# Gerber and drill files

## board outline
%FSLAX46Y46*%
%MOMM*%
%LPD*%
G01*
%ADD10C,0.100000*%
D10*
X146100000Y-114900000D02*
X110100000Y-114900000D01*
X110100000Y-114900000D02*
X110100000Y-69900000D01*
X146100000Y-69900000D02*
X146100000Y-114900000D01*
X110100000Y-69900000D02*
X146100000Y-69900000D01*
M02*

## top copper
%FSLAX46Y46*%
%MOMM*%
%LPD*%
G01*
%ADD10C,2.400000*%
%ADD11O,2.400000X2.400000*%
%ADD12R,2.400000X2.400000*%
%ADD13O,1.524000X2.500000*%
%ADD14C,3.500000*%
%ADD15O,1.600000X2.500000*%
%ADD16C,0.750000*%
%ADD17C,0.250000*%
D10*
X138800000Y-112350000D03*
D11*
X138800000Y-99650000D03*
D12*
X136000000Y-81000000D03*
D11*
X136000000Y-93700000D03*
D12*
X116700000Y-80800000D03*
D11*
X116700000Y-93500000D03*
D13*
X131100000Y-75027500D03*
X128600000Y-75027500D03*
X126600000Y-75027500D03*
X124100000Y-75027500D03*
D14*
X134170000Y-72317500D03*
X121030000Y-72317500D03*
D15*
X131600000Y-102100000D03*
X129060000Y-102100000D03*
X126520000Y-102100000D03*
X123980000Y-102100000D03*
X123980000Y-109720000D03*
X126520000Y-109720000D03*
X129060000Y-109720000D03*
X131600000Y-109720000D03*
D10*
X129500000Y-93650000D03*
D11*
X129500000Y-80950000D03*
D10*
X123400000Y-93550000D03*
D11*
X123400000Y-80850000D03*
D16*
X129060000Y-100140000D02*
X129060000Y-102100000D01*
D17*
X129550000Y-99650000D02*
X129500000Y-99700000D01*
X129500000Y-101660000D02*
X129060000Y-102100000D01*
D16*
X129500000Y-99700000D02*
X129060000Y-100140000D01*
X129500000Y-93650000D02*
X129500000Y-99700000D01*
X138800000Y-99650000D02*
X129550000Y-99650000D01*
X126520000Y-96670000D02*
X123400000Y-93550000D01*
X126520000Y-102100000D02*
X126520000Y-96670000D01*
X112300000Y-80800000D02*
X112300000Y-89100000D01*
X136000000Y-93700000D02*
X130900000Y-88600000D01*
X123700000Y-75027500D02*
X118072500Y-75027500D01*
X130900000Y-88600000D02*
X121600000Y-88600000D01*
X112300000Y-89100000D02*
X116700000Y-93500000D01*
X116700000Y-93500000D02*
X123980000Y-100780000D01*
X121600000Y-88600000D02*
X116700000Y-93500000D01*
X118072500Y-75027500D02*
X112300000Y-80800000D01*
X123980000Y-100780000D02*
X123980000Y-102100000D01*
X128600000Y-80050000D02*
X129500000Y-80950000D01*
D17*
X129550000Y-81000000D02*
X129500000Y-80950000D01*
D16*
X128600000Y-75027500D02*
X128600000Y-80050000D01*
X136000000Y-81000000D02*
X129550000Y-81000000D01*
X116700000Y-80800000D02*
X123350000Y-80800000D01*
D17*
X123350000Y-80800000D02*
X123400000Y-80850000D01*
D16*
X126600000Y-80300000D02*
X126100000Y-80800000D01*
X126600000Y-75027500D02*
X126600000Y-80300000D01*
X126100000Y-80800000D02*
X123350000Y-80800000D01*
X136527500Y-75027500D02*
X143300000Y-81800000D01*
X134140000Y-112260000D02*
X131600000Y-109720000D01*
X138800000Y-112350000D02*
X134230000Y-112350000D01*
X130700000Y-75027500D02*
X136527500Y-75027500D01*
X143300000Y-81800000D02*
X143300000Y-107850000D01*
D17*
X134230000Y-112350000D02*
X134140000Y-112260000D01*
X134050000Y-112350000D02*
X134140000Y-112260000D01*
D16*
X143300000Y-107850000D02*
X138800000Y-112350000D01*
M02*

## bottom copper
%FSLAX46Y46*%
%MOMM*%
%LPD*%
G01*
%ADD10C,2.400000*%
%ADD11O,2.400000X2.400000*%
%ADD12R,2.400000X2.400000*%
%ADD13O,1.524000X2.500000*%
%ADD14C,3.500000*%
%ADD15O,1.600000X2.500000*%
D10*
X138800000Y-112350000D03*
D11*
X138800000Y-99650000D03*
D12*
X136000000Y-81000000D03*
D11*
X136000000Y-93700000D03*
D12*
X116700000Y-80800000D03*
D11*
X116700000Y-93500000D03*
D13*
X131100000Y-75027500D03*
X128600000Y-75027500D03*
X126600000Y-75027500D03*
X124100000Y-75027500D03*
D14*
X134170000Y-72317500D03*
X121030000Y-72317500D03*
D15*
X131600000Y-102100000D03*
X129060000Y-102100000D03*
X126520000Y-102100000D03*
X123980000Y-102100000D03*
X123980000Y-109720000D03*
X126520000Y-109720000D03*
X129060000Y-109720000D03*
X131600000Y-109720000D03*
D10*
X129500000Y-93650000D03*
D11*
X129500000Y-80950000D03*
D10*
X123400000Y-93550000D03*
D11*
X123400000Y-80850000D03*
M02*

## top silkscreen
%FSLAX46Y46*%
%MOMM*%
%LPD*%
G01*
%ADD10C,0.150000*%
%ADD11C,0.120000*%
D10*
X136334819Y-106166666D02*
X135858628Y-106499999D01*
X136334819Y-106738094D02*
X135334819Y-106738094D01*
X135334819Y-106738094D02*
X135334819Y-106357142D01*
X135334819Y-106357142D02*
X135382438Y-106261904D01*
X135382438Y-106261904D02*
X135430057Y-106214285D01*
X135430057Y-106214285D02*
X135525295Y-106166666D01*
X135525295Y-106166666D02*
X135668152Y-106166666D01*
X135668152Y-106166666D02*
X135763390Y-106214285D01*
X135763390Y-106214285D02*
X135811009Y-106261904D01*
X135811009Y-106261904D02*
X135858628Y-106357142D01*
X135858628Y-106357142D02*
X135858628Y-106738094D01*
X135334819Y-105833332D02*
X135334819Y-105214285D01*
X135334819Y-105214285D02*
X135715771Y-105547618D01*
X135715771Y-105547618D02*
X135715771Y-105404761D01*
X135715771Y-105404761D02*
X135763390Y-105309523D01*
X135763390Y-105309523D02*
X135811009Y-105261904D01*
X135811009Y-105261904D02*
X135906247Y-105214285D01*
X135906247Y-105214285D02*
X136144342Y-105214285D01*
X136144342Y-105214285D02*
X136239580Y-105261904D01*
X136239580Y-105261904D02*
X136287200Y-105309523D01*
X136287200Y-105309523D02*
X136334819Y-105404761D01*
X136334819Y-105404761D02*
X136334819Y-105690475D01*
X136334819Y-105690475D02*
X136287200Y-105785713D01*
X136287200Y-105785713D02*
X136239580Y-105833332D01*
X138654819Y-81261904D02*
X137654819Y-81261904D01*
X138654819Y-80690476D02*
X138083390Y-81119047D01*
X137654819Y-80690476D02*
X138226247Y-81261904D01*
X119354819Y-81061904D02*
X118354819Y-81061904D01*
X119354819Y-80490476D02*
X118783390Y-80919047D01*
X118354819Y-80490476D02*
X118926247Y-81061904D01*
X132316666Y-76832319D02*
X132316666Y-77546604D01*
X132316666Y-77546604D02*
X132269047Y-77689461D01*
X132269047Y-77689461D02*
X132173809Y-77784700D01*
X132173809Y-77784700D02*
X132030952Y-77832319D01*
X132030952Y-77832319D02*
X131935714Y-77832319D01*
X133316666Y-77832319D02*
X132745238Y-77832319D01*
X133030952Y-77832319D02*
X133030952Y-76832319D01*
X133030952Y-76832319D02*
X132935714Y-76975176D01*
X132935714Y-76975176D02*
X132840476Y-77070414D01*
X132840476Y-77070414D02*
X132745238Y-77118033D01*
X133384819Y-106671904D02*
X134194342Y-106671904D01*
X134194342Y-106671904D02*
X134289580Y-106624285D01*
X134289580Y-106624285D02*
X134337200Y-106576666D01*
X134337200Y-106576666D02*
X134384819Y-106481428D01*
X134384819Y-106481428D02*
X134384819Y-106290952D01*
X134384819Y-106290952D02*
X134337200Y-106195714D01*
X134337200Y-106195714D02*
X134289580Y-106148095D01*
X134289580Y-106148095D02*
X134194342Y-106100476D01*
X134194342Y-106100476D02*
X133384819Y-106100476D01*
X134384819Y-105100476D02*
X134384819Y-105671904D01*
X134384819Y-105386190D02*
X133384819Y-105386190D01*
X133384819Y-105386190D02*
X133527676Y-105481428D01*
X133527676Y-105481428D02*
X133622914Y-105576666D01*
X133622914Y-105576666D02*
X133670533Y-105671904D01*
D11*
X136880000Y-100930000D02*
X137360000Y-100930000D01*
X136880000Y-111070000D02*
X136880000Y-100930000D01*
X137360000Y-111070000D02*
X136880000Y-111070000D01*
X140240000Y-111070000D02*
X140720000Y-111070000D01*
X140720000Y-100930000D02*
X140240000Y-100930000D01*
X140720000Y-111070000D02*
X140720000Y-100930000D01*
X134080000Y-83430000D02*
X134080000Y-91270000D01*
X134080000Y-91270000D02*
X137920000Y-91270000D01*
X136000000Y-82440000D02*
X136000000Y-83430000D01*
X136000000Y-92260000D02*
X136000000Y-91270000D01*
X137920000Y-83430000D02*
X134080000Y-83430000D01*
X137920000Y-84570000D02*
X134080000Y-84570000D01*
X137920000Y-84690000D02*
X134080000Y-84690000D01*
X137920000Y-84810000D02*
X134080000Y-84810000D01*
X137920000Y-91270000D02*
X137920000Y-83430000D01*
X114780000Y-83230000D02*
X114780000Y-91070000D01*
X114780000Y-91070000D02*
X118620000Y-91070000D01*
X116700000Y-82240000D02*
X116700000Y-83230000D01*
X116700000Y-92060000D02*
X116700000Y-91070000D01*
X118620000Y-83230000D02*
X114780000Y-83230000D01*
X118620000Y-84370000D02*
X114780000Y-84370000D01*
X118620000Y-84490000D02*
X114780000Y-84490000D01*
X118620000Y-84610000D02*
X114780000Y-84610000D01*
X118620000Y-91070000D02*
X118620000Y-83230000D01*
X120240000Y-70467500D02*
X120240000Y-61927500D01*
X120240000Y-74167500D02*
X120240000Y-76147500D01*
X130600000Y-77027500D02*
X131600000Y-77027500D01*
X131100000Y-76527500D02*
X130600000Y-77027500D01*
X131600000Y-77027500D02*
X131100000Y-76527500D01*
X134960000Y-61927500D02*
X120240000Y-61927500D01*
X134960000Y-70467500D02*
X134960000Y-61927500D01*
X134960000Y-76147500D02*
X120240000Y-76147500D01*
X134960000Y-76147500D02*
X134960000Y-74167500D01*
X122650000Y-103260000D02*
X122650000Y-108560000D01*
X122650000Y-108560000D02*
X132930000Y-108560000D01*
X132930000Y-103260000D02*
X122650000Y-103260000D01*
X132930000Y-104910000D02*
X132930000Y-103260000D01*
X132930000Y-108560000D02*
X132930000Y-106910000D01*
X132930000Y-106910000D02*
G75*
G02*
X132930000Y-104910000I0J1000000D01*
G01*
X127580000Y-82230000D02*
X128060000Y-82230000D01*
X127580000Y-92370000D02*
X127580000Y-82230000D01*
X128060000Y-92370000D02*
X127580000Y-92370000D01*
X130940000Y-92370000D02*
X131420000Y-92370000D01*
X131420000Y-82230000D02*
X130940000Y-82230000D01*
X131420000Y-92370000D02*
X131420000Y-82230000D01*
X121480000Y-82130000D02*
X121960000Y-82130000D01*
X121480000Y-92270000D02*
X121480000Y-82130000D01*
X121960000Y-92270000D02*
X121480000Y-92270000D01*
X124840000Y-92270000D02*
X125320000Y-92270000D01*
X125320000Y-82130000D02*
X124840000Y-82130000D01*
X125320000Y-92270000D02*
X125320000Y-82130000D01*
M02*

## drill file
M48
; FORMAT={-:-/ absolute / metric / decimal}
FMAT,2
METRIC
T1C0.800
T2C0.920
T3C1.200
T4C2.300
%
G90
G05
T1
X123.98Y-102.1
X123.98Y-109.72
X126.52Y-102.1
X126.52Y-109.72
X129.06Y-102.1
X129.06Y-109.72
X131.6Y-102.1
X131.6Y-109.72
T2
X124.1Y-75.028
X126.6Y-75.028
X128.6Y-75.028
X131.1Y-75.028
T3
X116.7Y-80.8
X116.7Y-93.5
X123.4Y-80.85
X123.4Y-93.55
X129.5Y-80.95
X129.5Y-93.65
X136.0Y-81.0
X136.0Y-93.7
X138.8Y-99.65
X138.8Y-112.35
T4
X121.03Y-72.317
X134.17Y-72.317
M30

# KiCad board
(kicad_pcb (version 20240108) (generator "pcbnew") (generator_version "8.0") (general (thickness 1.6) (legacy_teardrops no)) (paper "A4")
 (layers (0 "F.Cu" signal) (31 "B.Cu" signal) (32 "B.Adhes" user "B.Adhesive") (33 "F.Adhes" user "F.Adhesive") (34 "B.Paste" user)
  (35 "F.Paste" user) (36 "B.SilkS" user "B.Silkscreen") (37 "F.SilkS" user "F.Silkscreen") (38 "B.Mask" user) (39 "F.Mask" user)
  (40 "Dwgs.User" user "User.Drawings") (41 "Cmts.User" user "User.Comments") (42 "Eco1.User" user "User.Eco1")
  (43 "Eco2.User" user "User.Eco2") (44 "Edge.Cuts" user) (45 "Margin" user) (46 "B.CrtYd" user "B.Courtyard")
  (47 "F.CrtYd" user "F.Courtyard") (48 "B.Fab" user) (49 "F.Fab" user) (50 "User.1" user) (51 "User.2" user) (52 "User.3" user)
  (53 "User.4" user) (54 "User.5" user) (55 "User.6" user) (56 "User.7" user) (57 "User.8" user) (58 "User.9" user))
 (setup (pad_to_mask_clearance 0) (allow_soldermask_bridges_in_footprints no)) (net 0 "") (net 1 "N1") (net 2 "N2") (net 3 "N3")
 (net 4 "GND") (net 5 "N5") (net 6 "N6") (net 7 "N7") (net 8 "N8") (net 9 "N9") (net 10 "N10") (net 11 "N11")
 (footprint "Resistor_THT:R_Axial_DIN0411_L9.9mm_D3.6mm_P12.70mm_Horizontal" (layer "F.Cu") (at 138.8 112.35 90)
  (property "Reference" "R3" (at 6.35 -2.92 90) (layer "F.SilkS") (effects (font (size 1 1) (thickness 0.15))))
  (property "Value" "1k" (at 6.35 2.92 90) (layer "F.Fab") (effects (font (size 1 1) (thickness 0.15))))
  (fp_line (start 11.42 -1.92) (end 11.42 -1.44) (stroke (width 0.12) (type solid)) (layer "F.SilkS"))
  (fp_line (start 1.28 -1.92) (end 11.42 -1.92) (stroke (width 0.12) (type solid)) (layer "F.SilkS"))
  (fp_line (start 1.28 -1.44) (end 1.28 -1.92) (stroke (width 0.12) (type solid)) (layer "F.SilkS"))
  (fp_line (start 1.28 1.44) (end 1.28 1.92) (stroke (width 0.12) (type solid)) (layer "F.SilkS"))
  (fp_line (start 11.42 1.92) (end 11.42 1.44) (stroke (width 0.12) (type solid)) (layer "F.SilkS"))
  (fp_line (start 1.28 1.92) (end 11.42 1.92) (stroke (width 0.12) (type solid)) (layer "F.SilkS"))
  (pad "1" thru_hole circle (at 0 0 90) (size 2.4 2.4) (drill 1.2) (layers "*.Cu" "*.Mask") (remove_unused_layers no) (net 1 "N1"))
  (pad "2" thru_hole oval (at 12.7 0 90) (size 2.4 2.4) (drill 1.2) (layers "*.Cu" "*.Mask") (remove_unused_layers no) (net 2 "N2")))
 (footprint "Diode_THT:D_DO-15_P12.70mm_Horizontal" (layer "F.Cu") (at 136 81 -90)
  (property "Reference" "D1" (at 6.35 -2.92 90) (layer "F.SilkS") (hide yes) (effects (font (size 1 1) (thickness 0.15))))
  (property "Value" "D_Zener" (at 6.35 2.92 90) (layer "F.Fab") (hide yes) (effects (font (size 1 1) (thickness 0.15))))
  (fp_line (start 2.43 1.92) (end 10.27 1.92) (stroke (width 0.12) (type solid)) (layer "F.SilkS"))
  (fp_line (start 10.27 1.92) (end 10.27 -1.92) (stroke (width 0.12) (type solid)) (layer "F.SilkS"))
  (fp_line (start 1.44 0) (end 2.43 0) (stroke (width 0.12) (type solid)) (layer "F.SilkS"))
  (fp_line (start 11.26 0) (end 10.27 0) (stroke (width 0.12) (type solid)) (layer "F.SilkS"))
  (fp_line (start 2.43 -1.92) (end 2.43 1.92) (stroke (width 0.12) (type solid)) (layer "F.SilkS"))
  (fp_line (start 3.57 -1.92) (end 3.57 1.92) (stroke (width 0.12) (type solid)) (layer "F.SilkS"))
  (fp_line (start 3.69 -1.92) (end 3.69 1.92) (stroke (width 0.12) (type solid)) (layer "F.SilkS"))
  (fp_line (start 3.81 -1.92) (end 3.81 1.92) (stroke (width 0.12) (type solid)) (layer "F.SilkS"))
  (fp_line (start 10.27 -1.92) (end 2.43 -1.92) (stroke (width 0.12) (type solid)) (layer "F.SilkS"))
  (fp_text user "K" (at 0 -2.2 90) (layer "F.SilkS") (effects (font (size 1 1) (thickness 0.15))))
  (pad "1" thru_hole rect (at 0 0 270) (size 2.4 2.4) (drill 1.2) (layers "*.Cu" "*.Mask") (remove_unused_layers no) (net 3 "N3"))
  (pad "2" thru_hole oval (at 12.7 0 270) (size 2.4 2.4) (drill 1.2) (layers "*.Cu" "*.Mask") (remove_unused_layers no) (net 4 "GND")))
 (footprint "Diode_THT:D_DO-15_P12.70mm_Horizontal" (layer "F.Cu") (at 116.7 80.8 -90)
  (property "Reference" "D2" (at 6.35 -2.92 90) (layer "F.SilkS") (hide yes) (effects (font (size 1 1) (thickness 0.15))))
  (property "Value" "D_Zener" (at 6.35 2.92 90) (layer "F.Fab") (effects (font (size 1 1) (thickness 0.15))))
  (fp_line (start 2.43 1.92) (end 10.27 1.92) (stroke (width 0.12) (type solid)) (layer "F.SilkS"))
  (fp_line (start 10.27 1.92) (end 10.27 -1.92) (stroke (width 0.12) (type solid)) (layer "F.SilkS"))
  (fp_line (start 1.44 0) (end 2.43 0) (stroke (width 0.12) (type solid)) (layer "F.SilkS"))
  (fp_line (start 11.26 0) (end 10.27 0) (stroke (width 0.12) (type solid)) (layer "F.SilkS"))
  (fp_line (start 2.43 -1.92) (end 2.43 1.92) (stroke (width 0.12) (type solid)) (layer "F.SilkS"))
  (fp_line (start 3.57 -1.92) (end 3.57 1.92) (stroke (width 0.12) (type solid)) (layer "F.SilkS"))
  (fp_line (start 3.69 -1.92) (end 3.69 1.92) (stroke (width 0.12) (type solid)) (layer "F.SilkS"))
  (fp_line (start 3.81 -1.92) (end 3.81 1.92) (stroke (width 0.12) (type solid)) (layer "F.SilkS"))
  (fp_line (start 10.27 -1.92) (end 2.43 -1.92) (stroke (width 0.12) (type solid)) (layer "F.SilkS"))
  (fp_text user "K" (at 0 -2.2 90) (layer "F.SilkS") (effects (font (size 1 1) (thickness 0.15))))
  (pad "1" thru_hole rect (at 0 0 270) (size 2.4 2.4) (drill 1.2) (layers "*.Cu" "*.Mask") (remove_unused_layers no) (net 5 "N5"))
  (pad "2" thru_hole oval (at 12.7 0 270) (size 2.4 2.4) (drill 1.2) (layers "*.Cu" "*.Mask") (remove_unused_layers no) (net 4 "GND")))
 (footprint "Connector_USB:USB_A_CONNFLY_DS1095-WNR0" (layer "F.Cu") (at 131.1 75.0275 180)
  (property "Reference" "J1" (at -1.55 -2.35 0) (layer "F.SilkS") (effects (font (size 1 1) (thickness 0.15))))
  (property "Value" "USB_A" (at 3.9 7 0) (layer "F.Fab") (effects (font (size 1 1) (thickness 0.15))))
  (fp_line (start 10.86 4.56) (end 10.86 13.1) (stroke (width 0.12) (type solid)) (layer "F.SilkS"))
  (fp_line (start 10.86 0.86) (end 10.86 -1.12) (stroke (width 0.12) (type solid)) (layer "F.SilkS"))
  (fp_line (start 0.5 -2) (end -0.5 -2) (stroke (width 0.12) (type solid)) (layer "F.SilkS"))
  (fp_line (start 0 -1.5) (end 0.5 -2) (stroke (width 0.12) (type solid)) (layer "F.SilkS"))
  (fp_line (start -0.5 -2) (end 0 -1.5) (stroke (width 0.12) (type solid)) (layer "F.SilkS"))
  (fp_line (start -3.86 13.1) (end 10.86 13.1) (stroke (width 0.12) (type solid)) (layer "F.SilkS"))
  (fp_line (start -3.86 4.56) (end -3.86 13.1) (stroke (width 0.12) (type solid)) (layer "F.SilkS"))
  (fp_line (start -3.86 -1.12) (end 10.86 -1.12) (stroke (width 0.12) (type solid)) (layer "F.SilkS"))
  (fp_line (start -3.86 -1.12) (end -3.86 0.86) (stroke (width 0.12) (type solid)) (layer "F.SilkS"))
  (pad "1" thru_hole oval (at 0 0 180) (size 1.524 2.5) (drill 0.92) (layers "*.Cu" "*.Mask") (remove_unused_layers no) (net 1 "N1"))
  (pad "2" thru_hole oval (at 2.5 0 180) (size 1.524 2.5) (drill 0.92) (layers "*.Cu" "*.Mask") (remove_unused_layers no) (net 3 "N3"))
  (pad "3" thru_hole oval (at 4.5 0 180) (size 1.524 2.5) (drill 0.92) (layers "*.Cu" "*.Mask") (remove_unused_layers no) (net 5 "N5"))
  (pad "4" thru_hole oval (at 7 0 180) (size 1.524 2.5) (drill 0.92) (layers "*.Cu" "*.Mask") (remove_unused_layers no) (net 4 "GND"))
  (pad "5" thru_hole circle (at -3.07 2.71 180) (size 3.5 3.5) (drill 2.3) (layers "*.Cu" "*.Mask") (remove_unused_layers no) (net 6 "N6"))
  (pad "5" thru_hole circle (at 10.07 2.71 180) (size 3.5 3.5) (drill 2.3) (layers "*.Cu" "*.Mask") (remove_unused_layers no) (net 6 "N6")))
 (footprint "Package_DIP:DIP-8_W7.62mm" (layer "F.Cu") (at 131.6 102.1 -90)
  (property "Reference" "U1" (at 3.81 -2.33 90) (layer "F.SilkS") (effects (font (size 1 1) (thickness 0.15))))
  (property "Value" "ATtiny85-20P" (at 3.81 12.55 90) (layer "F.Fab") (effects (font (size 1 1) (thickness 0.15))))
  (fp_line (start 1.16 8.95) (end 6.46 8.95) (stroke (width 0.12) (type solid)) (layer "F.SilkS"))
  (fp_line (start 6.46 8.95) (end 6.46 -1.33) (stroke (width 0.12) (type solid)) (layer "F.SilkS"))
  (fp_line (start 1.16 -1.33) (end 1.16 8.95) (stroke (width 0.12) (type solid)) (layer "F.SilkS"))
  (fp_line (start 2.81 -1.33) (end 1.16 -1.33) (stroke (width 0.12) (type solid)) (layer "F.SilkS"))
  (fp_line (start 6.46 -1.33) (end 4.81 -1.33) (stroke (width 0.12) (type solid)) (layer "F.SilkS"))
  (fp_arc (start 4.81 -1.33) (mid 3.81 -0.33) (end 2.81 -1.33) (stroke (width 0.12) (type solid)) (layer "F.SilkS"))
  (pad "1" thru_hole oval (at 0 0 270) (size 2.5 1.6) (drill 0.8) (layers "*.Cu" "*.Mask") (remove_unused_layers no) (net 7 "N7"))
  (pad "2" thru_hole oval (at 0 2.54 270) (size 2.5 1.6) (drill 0.8) (layers "*.Cu" "*.Mask") (remove_unused_layers no) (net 2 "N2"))
  (pad "3" thru_hole oval (at 0 5.08 270) (size 2.5 1.6) (drill 0.8) (layers "*.Cu" "*.Mask") (remove_unused_layers no) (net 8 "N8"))
  (pad "4" thru_hole oval (at 0 7.62 270) (size 2.5 1.6) (drill 0.8) (layers "*.Cu" "*.Mask") (remove_unused_layers no) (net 4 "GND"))
  (pad "5" thru_hole oval (at 7.62 7.62 270) (size 2.5 1.6) (drill 0.8) (layers "*.Cu" "*.Mask") (remove_unused_layers no) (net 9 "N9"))
  (pad "6" thru_hole oval (at 7.62 5.08 270) (size 2.5 1.6) (drill 0.8) (layers "*.Cu" "*.Mask") (remove_unused_layers no) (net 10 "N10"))
  (pad "7" thru_hole oval (at 7.62 2.54 270) (size 2.5 1.6) (drill 0.8) (layers "*.Cu" "*.Mask") (remove_unused_layers no) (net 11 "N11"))
  (pad "8" thru_hole oval (at 7.62 0 270) (size 2.5 1.6) (drill 0.8) (layers "*.Cu" "*.Mask") (remove_unused_layers no) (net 1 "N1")))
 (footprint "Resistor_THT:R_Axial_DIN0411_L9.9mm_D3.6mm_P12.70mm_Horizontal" (layer "F.Cu") (at 129.5 93.65 90)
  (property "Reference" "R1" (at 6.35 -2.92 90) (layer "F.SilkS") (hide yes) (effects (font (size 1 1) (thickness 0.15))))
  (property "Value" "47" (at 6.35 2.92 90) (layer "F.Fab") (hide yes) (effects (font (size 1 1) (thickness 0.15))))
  (fp_line (start 11.42 -1.92) (end 11.42 -1.44) (stroke (width 0.12) (type solid)) (layer "F.SilkS"))
  (fp_line (start 1.28 -1.92) (end 11.42 -1.92) (stroke (width 0.12) (type solid)) (layer "F.SilkS"))
  (fp_line (start 1.28 -1.44) (end 1.28 -1.92) (stroke (width 0.12) (type solid)) (layer "F.SilkS"))
  (fp_line (start 1.28 1.44) (end 1.28 1.92) (stroke (width 0.12) (type solid)) (layer "F.SilkS"))
  (fp_line (start 11.42 1.92) (end 11.42 1.44) (stroke (width 0.12) (type solid)) (layer "F.SilkS"))
  (fp_line (start 1.28 1.92) (end 11.42 1.92) (stroke (width 0.12) (type solid)) (layer "F.SilkS"))
  (pad "1" thru_hole circle (at 0 0 90) (size 2.4 2.4) (drill 1.2) (layers "*.Cu" "*.Mask") (remove_unused_layers no) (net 2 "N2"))
  (pad "2" thru_hole oval (at 12.7 0 90) (size 2.4 2.4) (drill 1.2) (layers "*.Cu" "*.Mask") (remove_unused_layers no) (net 3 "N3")))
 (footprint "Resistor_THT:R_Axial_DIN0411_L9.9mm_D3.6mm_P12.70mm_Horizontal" (layer "F.Cu") (at 123.4 93.55 90)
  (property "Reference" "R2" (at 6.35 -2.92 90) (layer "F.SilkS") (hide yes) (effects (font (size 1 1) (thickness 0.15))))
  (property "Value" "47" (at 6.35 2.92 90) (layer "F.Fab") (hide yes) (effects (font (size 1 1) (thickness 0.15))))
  (fp_line (start 11.42 -1.92) (end 11.42 -1.44) (stroke (width 0.12) (type solid)) (layer "F.SilkS"))
  (fp_line (start 1.28 -1.92) (end 11.42 -1.92) (stroke (width 0.12) (type solid)) (layer "F.SilkS"))
  (fp_line (start 1.28 -1.44) (end 1.28 -1.92) (stroke (width 0.12) (type solid)) (layer "F.SilkS"))
  (fp_line (start 1.28 1.44) (end 1.28 1.92) (stroke (width 0.12) (type solid)) (layer "F.SilkS"))
  (fp_line (start 11.42 1.92) (end 11.42 1.44) (stroke (width 0.12) (type solid)) (layer "F.SilkS"))
  (fp_line (start 1.28 1.92) (end 11.42 1.92) (stroke (width 0.12) (type solid)) (layer "F.SilkS"))
  (pad "1" thru_hole circle (at 0 0 90) (size 2.4 2.4) (drill 1.2) (layers "*.Cu" "*.Mask") (remove_unused_layers no) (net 8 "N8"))
  (pad "2" thru_hole oval (at 12.7 0 90) (size 2.4 2.4) (drill 1.2) (layers "*.Cu" "*.Mask") (remove_unused_layers no) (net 5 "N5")))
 (gr_line (start 146.1 114.9) (end 110.1 114.9) (stroke (width 0.1) (type default)) (layer "Edge.Cuts"))
 (gr_line (start 110.1 114.9) (end 110.1 69.9) (stroke (width 0.1) (type default)) (layer "Edge.Cuts"))
 (gr_line (start 146.1 69.9) (end 146.1 114.9) (stroke (width 0.1) (type default)) (layer "Edge.Cuts"))
 (gr_line (start 110.1 69.9) (end 146.1 69.9) (stroke (width 0.1) (type default)) (layer "Edge.Cuts"))
 (segment (start 129.06 100.14) (end 129.06 102.1) (width 0.75) (layer "F.Cu") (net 2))
 (segment (start 129.55 99.65) (end 129.5 99.7) (width 0.25) (layer "F.Cu") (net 2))
 (segment (start 129.5 101.66) (end 129.06 102.1) (width 0.25) (layer "F.Cu") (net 2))
 (segment (start 129.5 99.7) (end 129.06 100.14) (width 0.75) (layer "F.Cu") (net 2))
 (segment (start 129.5 93.65) (end 129.5 99.7) (width 0.75) (layer "F.Cu") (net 2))
 (segment (start 138.8 99.65) (end 129.55 99.65) (width 0.75) (layer "F.Cu") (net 2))
 (segment (start 126.52 96.67) (end 123.4 93.55) (width 0.75) (layer "F.Cu") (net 8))
 (segment (start 126.52 102.1) (end 126.52 96.67) (width 0.75) (layer "F.Cu") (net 8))
 (segment (start 112.3 80.8) (end 112.3 89.1) (width 0.75) (layer "F.Cu") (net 4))
 (segment (start 136 93.7) (end 130.9 88.6) (width 0.75) (layer "F.Cu") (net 4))
 (segment (start 123.7 75.0275) (end 118.0725 75.0275) (width 0.75) (layer "F.Cu") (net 4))
 (segment (start 130.9 88.6) (end 121.6 88.6) (width 0.75) (layer "F.Cu") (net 4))
 (segment (start 112.3 89.1) (end 116.7 93.5) (width 0.75) (layer "F.Cu") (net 4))
 (segment (start 116.7 93.5) (end 123.98 100.78) (width 0.75) (layer "F.Cu") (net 4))
 (segment (start 121.6 88.6) (end 116.7 93.5) (width 0.75) (layer "F.Cu") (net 4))
 (segment (start 118.0725 75.0275) (end 112.3 80.8) (width 0.75) (layer "F.Cu") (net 4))
 (segment (start 123.98 100.78) (end 123.98 102.1) (width 0.75) (layer "F.Cu") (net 4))
 (segment (start 128.6 80.05) (end 129.5 80.95) (width 0.75) (layer "F.Cu") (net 3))
 (segment (start 129.55 81) (end 129.5 80.95) (width 0.25) (layer "F.Cu") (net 3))
 (segment (start 128.6 75.0275) (end 128.6 80.05) (width 0.75) (layer "F.Cu") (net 3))
 (segment (start 136 81) (end 129.55 81) (width 0.75) (layer "F.Cu") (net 3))
 (segment (start 116.7 80.8) (end 123.35 80.8) (width 0.75) (layer "F.Cu") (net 5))
 (segment (start 123.35 80.8) (end 123.4 80.85) (width 0.25) (layer "F.Cu") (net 5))
 (segment (start 126.6 80.3) (end 126.1 80.8) (width 0.75) (layer "F.Cu") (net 5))
 (segment (start 126.6 75.0275) (end 126.6 80.3) (width 0.75) (layer "F.Cu") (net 5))
 (segment (start 126.1 80.8) (end 123.35 80.8) (width 0.75) (layer "F.Cu") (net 5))
 (segment (start 136.5275 75.0275) (end 143.3 81.8) (width 0.75) (layer "F.Cu") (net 1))
 (segment (start 134.14 112.26) (end 131.6 109.72) (width 0.75) (layer "F.Cu") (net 1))
 (segment (start 138.8 112.35) (end 134.23 112.35) (width 0.75) (layer "F.Cu") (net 1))
 (segment (start 130.7 75.0275) (end 136.5275 75.0275) (width 0.75) (layer "F.Cu") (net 1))
 (segment (start 143.3 81.8) (end 143.3 107.85) (width 0.75) (layer "F.Cu") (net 1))
 (segment (start 134.23 112.35) (end 134.14 112.26) (width 0.25) (layer "F.Cu") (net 1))
 (segment (start 134.05 112.35) (end 134.14 112.26) (width 0.25) (layer "F.Cu") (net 1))
 (segment (start 143.3 107.85) (end 138.8 112.35) (width 0.75) (layer "F.Cu") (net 1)))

